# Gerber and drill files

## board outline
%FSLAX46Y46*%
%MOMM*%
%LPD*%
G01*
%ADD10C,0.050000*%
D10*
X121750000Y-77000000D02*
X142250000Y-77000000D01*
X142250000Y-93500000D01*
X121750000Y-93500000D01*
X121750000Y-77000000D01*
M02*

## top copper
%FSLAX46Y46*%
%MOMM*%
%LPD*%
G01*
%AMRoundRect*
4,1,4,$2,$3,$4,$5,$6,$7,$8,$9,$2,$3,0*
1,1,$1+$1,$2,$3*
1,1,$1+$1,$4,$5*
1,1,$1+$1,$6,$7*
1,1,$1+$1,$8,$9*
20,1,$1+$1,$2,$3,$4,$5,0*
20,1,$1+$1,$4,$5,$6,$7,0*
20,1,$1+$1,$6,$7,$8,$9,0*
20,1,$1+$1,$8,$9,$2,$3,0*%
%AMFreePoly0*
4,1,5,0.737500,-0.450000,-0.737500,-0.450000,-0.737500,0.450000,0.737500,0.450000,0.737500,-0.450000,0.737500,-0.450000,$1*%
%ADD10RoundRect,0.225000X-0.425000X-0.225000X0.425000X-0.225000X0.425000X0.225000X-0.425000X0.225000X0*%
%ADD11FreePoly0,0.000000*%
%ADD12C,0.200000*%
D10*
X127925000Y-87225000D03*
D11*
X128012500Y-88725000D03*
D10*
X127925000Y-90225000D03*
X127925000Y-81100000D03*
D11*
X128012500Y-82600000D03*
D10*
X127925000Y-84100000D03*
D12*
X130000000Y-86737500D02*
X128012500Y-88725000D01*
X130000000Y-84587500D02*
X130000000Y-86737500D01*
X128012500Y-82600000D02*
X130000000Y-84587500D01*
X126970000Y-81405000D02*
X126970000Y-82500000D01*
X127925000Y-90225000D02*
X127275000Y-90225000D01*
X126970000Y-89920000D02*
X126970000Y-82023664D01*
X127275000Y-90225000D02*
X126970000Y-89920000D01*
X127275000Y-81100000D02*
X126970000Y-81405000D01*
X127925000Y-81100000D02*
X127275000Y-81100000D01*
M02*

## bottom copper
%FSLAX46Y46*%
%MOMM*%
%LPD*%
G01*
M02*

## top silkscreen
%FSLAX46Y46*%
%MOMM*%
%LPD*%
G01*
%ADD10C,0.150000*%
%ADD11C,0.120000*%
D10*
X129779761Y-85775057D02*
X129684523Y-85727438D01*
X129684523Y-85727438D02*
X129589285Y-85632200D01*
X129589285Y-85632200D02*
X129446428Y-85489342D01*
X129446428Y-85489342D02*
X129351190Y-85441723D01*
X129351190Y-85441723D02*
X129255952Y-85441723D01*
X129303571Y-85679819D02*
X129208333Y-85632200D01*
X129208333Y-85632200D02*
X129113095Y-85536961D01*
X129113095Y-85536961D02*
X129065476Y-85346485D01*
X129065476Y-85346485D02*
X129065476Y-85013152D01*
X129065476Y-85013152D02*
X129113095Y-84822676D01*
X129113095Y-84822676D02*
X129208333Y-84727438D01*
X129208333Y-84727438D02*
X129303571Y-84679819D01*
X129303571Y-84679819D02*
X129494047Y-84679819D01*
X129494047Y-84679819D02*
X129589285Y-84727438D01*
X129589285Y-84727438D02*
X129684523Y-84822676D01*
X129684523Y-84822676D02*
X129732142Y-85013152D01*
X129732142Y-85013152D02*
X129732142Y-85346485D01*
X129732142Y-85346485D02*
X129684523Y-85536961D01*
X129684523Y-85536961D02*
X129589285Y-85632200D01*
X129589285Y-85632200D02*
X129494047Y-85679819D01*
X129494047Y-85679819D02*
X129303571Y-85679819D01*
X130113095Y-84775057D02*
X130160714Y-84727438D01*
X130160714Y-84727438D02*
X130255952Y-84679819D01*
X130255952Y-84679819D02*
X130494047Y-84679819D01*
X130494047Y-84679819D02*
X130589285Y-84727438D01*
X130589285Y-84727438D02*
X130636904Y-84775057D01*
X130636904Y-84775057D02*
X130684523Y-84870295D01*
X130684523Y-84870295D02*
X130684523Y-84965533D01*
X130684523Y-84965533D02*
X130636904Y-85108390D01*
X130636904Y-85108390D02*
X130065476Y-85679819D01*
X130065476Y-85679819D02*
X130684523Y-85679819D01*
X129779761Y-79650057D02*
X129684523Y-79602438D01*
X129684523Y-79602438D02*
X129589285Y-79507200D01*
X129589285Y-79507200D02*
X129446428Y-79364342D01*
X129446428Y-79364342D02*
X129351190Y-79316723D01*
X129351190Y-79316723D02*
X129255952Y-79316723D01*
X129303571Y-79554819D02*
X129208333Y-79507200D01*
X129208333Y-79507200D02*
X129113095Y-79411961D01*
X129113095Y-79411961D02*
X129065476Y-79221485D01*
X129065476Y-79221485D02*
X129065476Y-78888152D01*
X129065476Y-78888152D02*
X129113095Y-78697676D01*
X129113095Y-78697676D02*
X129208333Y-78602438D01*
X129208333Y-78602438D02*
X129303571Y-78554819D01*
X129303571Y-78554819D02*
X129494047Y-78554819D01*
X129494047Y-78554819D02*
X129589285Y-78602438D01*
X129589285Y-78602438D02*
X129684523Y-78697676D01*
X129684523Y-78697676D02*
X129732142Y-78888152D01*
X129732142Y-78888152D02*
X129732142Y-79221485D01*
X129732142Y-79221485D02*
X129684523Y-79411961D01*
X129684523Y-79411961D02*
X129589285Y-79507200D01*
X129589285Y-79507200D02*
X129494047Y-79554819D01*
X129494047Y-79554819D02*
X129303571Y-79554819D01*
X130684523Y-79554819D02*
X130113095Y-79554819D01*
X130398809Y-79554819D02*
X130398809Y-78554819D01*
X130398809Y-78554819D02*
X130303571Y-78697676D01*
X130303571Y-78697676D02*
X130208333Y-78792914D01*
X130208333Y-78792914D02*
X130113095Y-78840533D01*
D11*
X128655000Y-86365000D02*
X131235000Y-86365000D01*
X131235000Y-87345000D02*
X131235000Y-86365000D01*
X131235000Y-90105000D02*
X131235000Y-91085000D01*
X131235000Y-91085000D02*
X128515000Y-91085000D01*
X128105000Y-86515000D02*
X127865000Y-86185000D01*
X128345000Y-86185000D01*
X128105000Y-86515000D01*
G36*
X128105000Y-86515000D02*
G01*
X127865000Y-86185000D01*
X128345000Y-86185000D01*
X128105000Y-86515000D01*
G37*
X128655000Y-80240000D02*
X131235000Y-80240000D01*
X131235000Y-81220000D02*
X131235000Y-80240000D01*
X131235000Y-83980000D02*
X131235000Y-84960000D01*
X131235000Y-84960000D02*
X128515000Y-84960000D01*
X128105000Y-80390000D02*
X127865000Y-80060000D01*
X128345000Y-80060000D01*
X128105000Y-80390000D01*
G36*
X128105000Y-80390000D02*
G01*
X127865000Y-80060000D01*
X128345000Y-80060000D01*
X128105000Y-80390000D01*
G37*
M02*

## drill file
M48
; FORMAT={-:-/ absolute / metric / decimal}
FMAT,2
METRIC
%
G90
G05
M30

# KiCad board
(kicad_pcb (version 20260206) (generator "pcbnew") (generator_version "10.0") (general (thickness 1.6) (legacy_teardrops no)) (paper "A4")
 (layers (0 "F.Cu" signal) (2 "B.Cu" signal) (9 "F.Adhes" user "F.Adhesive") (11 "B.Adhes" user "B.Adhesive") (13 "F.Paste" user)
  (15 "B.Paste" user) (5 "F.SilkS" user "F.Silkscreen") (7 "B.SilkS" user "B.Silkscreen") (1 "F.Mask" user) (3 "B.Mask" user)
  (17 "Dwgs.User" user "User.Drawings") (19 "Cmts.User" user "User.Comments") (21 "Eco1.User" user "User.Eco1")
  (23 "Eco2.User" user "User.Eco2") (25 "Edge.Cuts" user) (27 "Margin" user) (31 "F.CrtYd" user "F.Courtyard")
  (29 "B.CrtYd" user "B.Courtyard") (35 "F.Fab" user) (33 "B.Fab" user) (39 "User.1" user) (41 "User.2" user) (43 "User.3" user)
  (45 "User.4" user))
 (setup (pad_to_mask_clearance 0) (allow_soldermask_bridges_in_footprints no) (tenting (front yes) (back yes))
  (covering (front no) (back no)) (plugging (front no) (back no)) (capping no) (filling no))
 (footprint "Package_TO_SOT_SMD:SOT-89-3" (layer "F.Cu") (at 129.875 88.725)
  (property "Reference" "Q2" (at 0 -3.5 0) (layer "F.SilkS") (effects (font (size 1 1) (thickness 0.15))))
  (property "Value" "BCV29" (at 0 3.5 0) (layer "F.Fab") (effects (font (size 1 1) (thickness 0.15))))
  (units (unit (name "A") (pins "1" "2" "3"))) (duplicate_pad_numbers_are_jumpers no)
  (fp_line (start -1.22 -2.36) (end 1.36 -2.36) (stroke (width 0.12) (type solid)) (layer "F.SilkS"))
  (fp_line (start 1.36 -1.38) (end 1.36 -2.36) (stroke (width 0.12) (type solid)) (layer "F.SilkS"))
  (fp_line (start 1.36 1.38) (end 1.36 2.36) (stroke (width 0.12) (type solid)) (layer "F.SilkS"))
  (fp_line (start 1.36 2.36) (end -1.36 2.36) (stroke (width 0.12) (type solid)) (layer "F.SilkS"))
  (fp_poly
   (pts (xy -1.77 -2.21) (xy -2.01 -2.54) (xy -1.53 -2.54) (xy -1.77 -2.21)) (stroke (width 0.12) (type solid)) (fill yes) (layer "F.SilkS"))
  (pad "1" smd roundrect (at -1.95 -1.5) (size 1.3 0.9) (layers "F.Cu" "F.Mask" "F.Paste") (roundrect_rratio 0.25) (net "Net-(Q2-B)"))
  (pad "2" smd custom (at -1.8625 0) (size 1.475 0.9) (layers "F.Cu" "F.Mask" "F.Paste") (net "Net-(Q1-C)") (zone_connect 2)
   (thermal_bridge_angle 45) (options (clearance outline) (anchor rect)) (primitives))
  (pad "3" smd roundrect (at -1.95 1.5) (size 1.3 0.9) (layers "F.Cu" "F.Mask" "F.Paste") (roundrect_rratio 0.25) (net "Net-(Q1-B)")))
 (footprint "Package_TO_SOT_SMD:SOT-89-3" (layer "F.Cu") (at 129.875 82.6)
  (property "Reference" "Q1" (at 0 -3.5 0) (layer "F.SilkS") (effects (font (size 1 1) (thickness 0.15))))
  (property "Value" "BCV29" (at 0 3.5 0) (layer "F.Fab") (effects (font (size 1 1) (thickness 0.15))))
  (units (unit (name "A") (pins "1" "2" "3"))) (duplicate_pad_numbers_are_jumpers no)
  (fp_line (start -1.22 -2.36) (end 1.36 -2.36) (stroke (width 0.12) (type solid)) (layer "F.SilkS"))
  (fp_line (start 1.36 -1.38) (end 1.36 -2.36) (stroke (width 0.12) (type solid)) (layer "F.SilkS"))
  (fp_line (start 1.36 1.38) (end 1.36 2.36) (stroke (width 0.12) (type solid)) (layer "F.SilkS"))
  (fp_line (start 1.36 2.36) (end -1.36 2.36) (stroke (width 0.12) (type solid)) (layer "F.SilkS"))
  (fp_poly
   (pts (xy -1.77 -2.21) (xy -2.01 -2.54) (xy -1.53 -2.54) (xy -1.77 -2.21)) (stroke (width 0.12) (type solid)) (fill yes) (layer "F.SilkS"))
  (pad "1" smd roundrect (at -1.95 -1.5) (size 1.3 0.9) (layers "F.Cu" "F.Mask" "F.Paste") (roundrect_rratio 0.25) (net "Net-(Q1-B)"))
  (pad "2" smd custom (at -1.8625 0) (size 1.475 0.9) (layers "F.Cu" "F.Mask" "F.Paste") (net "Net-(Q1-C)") (zone_connect 2)
   (thermal_bridge_angle 45) (options (clearance outline) (anchor rect)) (primitives))
  (pad "3" smd roundrect (at -1.95 1.5) (size 1.3 0.9) (layers "F.Cu" "F.Mask" "F.Paste") (roundrect_rratio 0.25) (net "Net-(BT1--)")))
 (gr_rect (start 121.75 77) (end 142.25 93.5) (stroke (width 0.05) (type default)) (fill no) (layer "Edge.Cuts"))
 (segment (start 130 86.7375) (end 128.0125 88.725) (width 0.2) (layer "F.Cu") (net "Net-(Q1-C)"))
 (segment (start 130 84.5875) (end 130 86.7375) (width 0.2) (layer "F.Cu") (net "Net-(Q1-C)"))
 (segment (start 128.0125 82.6) (end 130 84.5875) (width 0.2) (layer "F.Cu") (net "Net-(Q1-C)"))
 (segment (start 126.97 81.405) (end 126.97 82.5) (width 0.2) (layer "F.Cu") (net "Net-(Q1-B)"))
 (segment (start 127.925 90.225) (end 127.275 90.225) (width 0.2) (layer "F.Cu") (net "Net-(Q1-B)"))
 (segment (start 126.97 89.92) (end 126.97 82.023664) (width 0.2) (layer "F.Cu") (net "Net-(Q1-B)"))
 (segment (start 127.275 90.225) (end 126.97 89.92) (width 0.2) (layer "F.Cu") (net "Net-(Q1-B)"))
 (segment (start 127.275 81.1) (end 126.97 81.405) (width 0.2) (layer "F.Cu") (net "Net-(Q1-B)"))
 (segment (start 127.925 81.1) (end 127.275 81.1) (width 0.2) (layer "F.Cu") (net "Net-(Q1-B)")))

